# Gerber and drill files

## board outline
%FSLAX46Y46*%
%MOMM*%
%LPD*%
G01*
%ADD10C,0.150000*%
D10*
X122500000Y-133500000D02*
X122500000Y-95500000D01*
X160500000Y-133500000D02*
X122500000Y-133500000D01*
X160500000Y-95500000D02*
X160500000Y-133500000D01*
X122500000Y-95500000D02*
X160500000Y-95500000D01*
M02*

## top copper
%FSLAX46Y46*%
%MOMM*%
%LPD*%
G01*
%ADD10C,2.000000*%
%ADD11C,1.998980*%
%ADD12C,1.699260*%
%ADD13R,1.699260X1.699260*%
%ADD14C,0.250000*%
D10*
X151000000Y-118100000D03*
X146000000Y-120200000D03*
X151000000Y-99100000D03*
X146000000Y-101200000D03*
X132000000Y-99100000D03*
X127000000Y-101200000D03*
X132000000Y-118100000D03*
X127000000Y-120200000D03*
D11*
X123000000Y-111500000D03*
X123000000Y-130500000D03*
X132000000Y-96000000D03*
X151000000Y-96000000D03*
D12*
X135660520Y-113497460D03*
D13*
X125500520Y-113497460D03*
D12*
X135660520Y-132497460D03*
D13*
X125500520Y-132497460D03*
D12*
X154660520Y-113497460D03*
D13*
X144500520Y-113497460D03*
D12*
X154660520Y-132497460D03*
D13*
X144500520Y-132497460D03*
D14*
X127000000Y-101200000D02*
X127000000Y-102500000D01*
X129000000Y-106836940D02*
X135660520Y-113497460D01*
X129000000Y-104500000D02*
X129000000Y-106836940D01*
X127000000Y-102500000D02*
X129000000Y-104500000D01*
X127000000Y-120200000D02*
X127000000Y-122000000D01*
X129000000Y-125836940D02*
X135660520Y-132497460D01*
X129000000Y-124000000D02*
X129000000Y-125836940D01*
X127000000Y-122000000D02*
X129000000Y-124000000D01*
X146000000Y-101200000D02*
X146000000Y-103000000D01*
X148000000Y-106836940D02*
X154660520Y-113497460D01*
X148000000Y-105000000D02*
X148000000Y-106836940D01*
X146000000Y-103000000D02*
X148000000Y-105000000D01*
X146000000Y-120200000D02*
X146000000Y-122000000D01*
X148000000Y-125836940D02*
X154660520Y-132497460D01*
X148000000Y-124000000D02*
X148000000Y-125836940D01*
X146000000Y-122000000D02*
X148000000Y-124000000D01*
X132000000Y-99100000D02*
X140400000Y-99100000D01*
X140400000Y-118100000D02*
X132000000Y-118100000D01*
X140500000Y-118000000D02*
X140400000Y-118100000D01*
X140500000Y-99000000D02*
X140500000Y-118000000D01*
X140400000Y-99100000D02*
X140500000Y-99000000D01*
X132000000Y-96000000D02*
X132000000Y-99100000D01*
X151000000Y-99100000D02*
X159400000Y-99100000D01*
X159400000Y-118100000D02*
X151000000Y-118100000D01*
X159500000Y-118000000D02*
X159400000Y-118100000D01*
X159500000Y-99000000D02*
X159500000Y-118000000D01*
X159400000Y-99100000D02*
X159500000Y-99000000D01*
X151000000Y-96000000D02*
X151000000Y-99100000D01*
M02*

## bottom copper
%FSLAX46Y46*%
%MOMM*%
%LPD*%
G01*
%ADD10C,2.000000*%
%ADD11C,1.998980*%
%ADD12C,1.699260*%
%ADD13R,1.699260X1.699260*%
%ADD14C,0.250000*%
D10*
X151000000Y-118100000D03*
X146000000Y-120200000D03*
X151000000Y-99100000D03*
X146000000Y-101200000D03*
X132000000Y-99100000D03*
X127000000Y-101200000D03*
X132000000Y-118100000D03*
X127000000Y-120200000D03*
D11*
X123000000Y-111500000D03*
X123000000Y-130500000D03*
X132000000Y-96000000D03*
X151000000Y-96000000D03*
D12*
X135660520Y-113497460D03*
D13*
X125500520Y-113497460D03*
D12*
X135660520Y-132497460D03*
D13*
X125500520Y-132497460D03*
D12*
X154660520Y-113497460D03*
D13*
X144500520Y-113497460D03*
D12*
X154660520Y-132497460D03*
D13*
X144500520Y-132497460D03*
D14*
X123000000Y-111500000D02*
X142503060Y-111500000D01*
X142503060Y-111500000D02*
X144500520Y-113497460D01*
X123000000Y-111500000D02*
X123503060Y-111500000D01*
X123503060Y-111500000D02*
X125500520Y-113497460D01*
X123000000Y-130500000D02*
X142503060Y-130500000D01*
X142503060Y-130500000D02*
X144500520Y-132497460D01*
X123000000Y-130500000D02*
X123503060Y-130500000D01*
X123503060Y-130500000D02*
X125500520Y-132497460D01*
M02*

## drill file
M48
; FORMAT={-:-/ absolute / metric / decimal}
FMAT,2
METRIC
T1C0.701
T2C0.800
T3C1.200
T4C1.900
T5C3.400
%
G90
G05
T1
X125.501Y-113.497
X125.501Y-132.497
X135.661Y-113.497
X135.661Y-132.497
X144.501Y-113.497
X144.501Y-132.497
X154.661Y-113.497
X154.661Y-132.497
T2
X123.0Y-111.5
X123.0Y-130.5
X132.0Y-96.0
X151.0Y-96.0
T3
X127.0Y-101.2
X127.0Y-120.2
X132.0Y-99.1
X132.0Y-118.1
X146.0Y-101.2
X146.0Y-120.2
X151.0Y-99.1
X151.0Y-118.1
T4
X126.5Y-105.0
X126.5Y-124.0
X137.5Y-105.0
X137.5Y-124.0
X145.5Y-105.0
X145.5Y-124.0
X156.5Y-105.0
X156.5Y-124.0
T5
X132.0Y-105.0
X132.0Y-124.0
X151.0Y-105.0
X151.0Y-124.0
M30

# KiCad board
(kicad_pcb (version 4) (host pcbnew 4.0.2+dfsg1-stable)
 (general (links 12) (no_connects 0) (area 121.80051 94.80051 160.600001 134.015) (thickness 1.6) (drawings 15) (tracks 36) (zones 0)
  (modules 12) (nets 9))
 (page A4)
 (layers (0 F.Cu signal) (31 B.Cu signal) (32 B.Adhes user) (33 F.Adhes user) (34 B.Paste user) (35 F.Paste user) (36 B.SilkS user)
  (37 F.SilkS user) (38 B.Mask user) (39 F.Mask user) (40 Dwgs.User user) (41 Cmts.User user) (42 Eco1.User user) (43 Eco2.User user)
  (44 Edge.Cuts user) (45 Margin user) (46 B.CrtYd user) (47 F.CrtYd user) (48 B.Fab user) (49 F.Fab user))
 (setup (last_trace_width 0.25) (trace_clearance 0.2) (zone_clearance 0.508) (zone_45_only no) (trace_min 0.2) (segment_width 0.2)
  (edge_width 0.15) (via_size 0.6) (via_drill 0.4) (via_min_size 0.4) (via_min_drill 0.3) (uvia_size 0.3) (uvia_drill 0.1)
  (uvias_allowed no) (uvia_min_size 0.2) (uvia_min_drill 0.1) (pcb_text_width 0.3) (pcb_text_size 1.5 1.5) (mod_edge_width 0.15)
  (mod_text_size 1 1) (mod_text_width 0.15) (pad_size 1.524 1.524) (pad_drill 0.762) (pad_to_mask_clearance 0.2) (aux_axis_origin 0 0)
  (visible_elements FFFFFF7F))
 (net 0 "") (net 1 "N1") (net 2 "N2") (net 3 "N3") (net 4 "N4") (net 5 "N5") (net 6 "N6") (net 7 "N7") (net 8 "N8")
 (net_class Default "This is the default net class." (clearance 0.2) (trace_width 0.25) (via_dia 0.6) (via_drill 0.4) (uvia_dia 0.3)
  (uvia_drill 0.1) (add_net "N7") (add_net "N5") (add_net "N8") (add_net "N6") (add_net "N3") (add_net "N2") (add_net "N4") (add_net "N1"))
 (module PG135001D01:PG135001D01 (layer F.Cu) (at 151 124)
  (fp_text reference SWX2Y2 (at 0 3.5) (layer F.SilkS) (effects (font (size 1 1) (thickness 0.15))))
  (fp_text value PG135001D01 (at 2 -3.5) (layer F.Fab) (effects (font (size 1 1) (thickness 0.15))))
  (pad "" np_thru_hole circle (at 0 0) (size 3.4 3.4) (drill 3.4) (layers *.Cu *.Mask F.SilkS))
  (pad "" np_thru_hole circle (at 5.5 0) (size 1.9 1.9) (drill 1.9) (layers *.Cu *.Mask F.SilkS))
  (pad "" np_thru_hole circle (at -5.5 0) (size 1.9 1.9) (drill 1.9) (layers *.Cu *.Mask F.SilkS))
  (pad 1 thru_hole circle (at 0 -5.9) (size 2 2) (drill 1.2) (layers *.Cu *.Mask F.SilkS) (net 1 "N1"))
  (pad 2 thru_hole circle (at -5 -3.8) (size 2 2) (drill 1.2) (layers *.Cu *.Mask F.SilkS) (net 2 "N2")))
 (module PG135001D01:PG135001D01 (layer F.Cu) (at 151 105)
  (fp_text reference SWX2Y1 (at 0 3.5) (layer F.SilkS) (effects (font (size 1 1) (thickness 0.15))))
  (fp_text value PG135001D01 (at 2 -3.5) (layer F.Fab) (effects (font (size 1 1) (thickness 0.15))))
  (pad "" np_thru_hole circle (at 0 0) (size 3.4 3.4) (drill 3.4) (layers *.Cu *.Mask F.SilkS))
  (pad "" np_thru_hole circle (at 5.5 0) (size 1.9 1.9) (drill 1.9) (layers *.Cu *.Mask F.SilkS))
  (pad "" np_thru_hole circle (at -5.5 0) (size 1.9 1.9) (drill 1.9) (layers *.Cu *.Mask F.SilkS))
  (pad 1 thru_hole circle (at 0 -5.9) (size 2 2) (drill 1.2) (layers *.Cu *.Mask F.SilkS) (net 1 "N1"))
  (pad 2 thru_hole circle (at -5 -3.8) (size 2 2) (drill 1.2) (layers *.Cu *.Mask F.SilkS) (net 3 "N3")))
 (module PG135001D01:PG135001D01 (layer F.Cu) (at 132 105)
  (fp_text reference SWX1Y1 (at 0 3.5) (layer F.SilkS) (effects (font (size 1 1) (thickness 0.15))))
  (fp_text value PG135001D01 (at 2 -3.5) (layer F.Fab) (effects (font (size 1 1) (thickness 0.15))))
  (pad "" np_thru_hole circle (at 0 0) (size 3.4 3.4) (drill 3.4) (layers *.Cu *.Mask F.SilkS))
  (pad "" np_thru_hole circle (at 5.5 0) (size 1.9 1.9) (drill 1.9) (layers *.Cu *.Mask F.SilkS))
  (pad "" np_thru_hole circle (at -5.5 0) (size 1.9 1.9) (drill 1.9) (layers *.Cu *.Mask F.SilkS))
  (pad 1 thru_hole circle (at 0 -5.9) (size 2 2) (drill 1.2) (layers *.Cu *.Mask F.SilkS) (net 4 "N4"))
  (pad 2 thru_hole circle (at -5 -3.8) (size 2 2) (drill 1.2) (layers *.Cu *.Mask F.SilkS) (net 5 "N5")))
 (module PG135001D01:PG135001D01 (layer F.Cu) (at 132 124)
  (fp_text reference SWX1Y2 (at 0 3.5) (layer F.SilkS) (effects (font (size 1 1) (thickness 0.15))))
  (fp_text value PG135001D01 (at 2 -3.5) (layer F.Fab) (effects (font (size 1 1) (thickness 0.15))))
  (pad "" np_thru_hole circle (at 0 0) (size 3.4 3.4) (drill 3.4) (layers *.Cu *.Mask F.SilkS))
  (pad "" np_thru_hole circle (at 5.5 0) (size 1.9 1.9) (drill 1.9) (layers *.Cu *.Mask F.SilkS))
  (pad "" np_thru_hole circle (at -5.5 0) (size 1.9 1.9) (drill 1.9) (layers *.Cu *.Mask F.SilkS))
  (pad 1 thru_hole circle (at 0 -5.9) (size 2 2) (drill 1.2) (layers *.Cu *.Mask F.SilkS) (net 4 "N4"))
  (pad 2 thru_hole circle (at -5 -3.8) (size 2 2) (drill 1.2) (layers *.Cu *.Mask F.SilkS) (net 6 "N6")))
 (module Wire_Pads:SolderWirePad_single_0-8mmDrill (layer F.Cu) (at 123 111.5)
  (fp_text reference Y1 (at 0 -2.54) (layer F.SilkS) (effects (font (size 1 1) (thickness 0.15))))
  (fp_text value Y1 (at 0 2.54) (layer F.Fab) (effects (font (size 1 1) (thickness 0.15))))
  (pad 1 thru_hole circle (at 0 0) (size 1.99898 1.99898) (drill 0.8001) (layers *.Cu *.Mask F.SilkS) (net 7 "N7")))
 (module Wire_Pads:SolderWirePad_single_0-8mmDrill (layer F.Cu) (at 123 130.5)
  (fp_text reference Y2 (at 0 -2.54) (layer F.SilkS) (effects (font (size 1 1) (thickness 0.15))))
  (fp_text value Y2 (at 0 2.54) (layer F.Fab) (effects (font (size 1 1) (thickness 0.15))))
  (pad 1 thru_hole circle (at 0 0) (size 1.99898 1.99898) (drill 0.8001) (layers *.Cu *.Mask F.SilkS) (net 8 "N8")))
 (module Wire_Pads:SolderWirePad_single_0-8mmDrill (layer F.Cu) (at 132 96)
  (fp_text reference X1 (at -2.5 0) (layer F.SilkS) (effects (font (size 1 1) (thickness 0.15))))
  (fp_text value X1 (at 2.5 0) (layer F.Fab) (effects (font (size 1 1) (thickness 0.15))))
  (pad 1 thru_hole circle (at 0 0) (size 1.99898 1.99898) (drill 0.8001) (layers *.Cu *.Mask F.SilkS) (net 4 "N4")))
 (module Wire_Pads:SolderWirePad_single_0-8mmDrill (layer F.Cu) (at 151 96)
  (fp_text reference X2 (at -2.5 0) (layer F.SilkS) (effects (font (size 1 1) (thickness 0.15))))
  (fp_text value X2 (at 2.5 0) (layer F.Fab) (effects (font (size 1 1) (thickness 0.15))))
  (pad 1 thru_hole circle (at 0 0) (size 1.99898 1.99898) (drill 0.8001) (layers *.Cu *.Mask F.SilkS) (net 1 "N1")))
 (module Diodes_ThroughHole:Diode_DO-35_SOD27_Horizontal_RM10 (layer F.Cu) (at 125.5 113.5)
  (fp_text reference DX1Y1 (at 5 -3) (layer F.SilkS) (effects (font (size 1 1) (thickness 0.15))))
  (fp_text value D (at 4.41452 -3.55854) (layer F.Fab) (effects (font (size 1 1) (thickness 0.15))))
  (pad 2 thru_hole circle (at 10.16052 -0.00254 180) (size 1.69926 1.69926) (drill 0.70104) (layers *.Cu *.Mask F.SilkS) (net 5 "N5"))
  (pad 1 thru_hole rect (at 0.00052 -0.00254 180) (size 1.69926 1.69926) (drill 0.70104) (layers *.Cu *.Mask F.SilkS) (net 7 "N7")))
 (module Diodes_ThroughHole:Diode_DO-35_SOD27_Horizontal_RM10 (layer F.Cu) (at 125.5 132.5)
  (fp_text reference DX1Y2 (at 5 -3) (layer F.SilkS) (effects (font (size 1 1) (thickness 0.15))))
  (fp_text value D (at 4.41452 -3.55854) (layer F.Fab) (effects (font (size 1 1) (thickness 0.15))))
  (pad 2 thru_hole circle (at 10.16052 -0.00254 180) (size 1.69926 1.69926) (drill 0.70104) (layers *.Cu *.Mask F.SilkS) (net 6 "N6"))
  (pad 1 thru_hole rect (at 0.00052 -0.00254 180) (size 1.69926 1.69926) (drill 0.70104) (layers *.Cu *.Mask F.SilkS) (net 8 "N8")))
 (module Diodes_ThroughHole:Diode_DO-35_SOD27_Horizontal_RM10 (layer F.Cu) (at 144.5 113.5)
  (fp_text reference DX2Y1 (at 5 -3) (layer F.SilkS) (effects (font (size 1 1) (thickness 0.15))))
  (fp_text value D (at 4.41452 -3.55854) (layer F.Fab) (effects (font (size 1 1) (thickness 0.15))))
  (pad 2 thru_hole circle (at 10.16052 -0.00254 180) (size 1.69926 1.69926) (drill 0.70104) (layers *.Cu *.Mask F.SilkS) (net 3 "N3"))
  (pad 1 thru_hole rect (at 0.00052 -0.00254 180) (size 1.69926 1.69926) (drill 0.70104) (layers *.Cu *.Mask F.SilkS) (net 7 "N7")))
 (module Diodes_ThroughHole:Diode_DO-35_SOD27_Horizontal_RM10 (layer F.Cu) (at 144.5 132.5)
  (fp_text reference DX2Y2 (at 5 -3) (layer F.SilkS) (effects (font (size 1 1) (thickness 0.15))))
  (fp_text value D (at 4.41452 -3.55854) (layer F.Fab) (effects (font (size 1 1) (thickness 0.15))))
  (pad 2 thru_hole circle (at 10.16052 -0.00254 180) (size 1.69926 1.69926) (drill 0.70104) (layers *.Cu *.Mask F.SilkS) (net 2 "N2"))
  (pad 1 thru_hole rect (at 0.00052 -0.00254 180) (size 1.69926 1.69926) (drill 0.70104) (layers *.Cu *.Mask F.SilkS) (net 8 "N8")))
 (gr_line (start 122.5 133.5) (end 122.5 95.5) (angle 90) (layer Edge.Cuts) (width 0.15))
 (gr_line (start 160.5 133.5) (end 122.5 133.5) (angle 90) (layer Edge.Cuts) (width 0.15))
 (gr_line (start 160.5 95.5) (end 160.5 133.5) (angle 90) (layer Edge.Cuts) (width 0.15))
 (gr_line (start 122.5 95.5) (end 160.5 95.5) (angle 90) (layer Edge.Cuts) (width 0.15))
 (segment (start 127 101.2) (end 127 102.5) (width 0.25) (layer F.Cu) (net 5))
 (segment (start 129 106.83694) (end 135.66052 113.49746) (width 0.25) (layer F.Cu) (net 5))
 (segment (start 129 104.5) (end 129 106.83694) (width 0.25) (layer F.Cu) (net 5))
 (segment (start 127 102.5) (end 129 104.5) (width 0.25) (layer F.Cu) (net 5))
 (segment (start 123 111.5) (end 142.50306 111.5) (width 0.25) (layer B.Cu) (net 7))
 (segment (start 142.50306 111.5) (end 144.50052 113.49746) (width 0.25) (layer B.Cu) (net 7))
 (segment (start 123 111.5) (end 123.50306 111.5) (width 0.25) (layer B.Cu) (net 7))
 (segment (start 123.50306 111.5) (end 125.50052 113.49746) (width 0.25) (layer B.Cu) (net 7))
 (segment (start 127 120.2) (end 127 122) (width 0.25) (layer F.Cu) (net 6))
 (segment (start 129 125.83694) (end 135.66052 132.49746) (width 0.25) (layer F.Cu) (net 6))
 (segment (start 129 124) (end 129 125.83694) (width 0.25) (layer F.Cu) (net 6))
 (segment (start 127 122) (end 129 124) (width 0.25) (layer F.Cu) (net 6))
 (segment (start 123 130.5) (end 142.50306 130.5) (width 0.25) (layer B.Cu) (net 8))
 (segment (start 142.50306 130.5) (end 144.50052 132.49746) (width 0.25) (layer B.Cu) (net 8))
 (segment (start 123 130.5) (end 123.50306 130.5) (width 0.25) (layer B.Cu) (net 8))
 (segment (start 123.50306 130.5) (end 125.50052 132.49746) (width 0.25) (layer B.Cu) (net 8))
 (segment (start 146 101.2) (end 146 103) (width 0.25) (layer F.Cu) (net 3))
 (segment (start 148 106.83694) (end 154.66052 113.49746) (width 0.25) (layer F.Cu) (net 3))
 (segment (start 148 105) (end 148 106.83694) (width 0.25) (layer F.Cu) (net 3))
 (segment (start 146 103) (end 148 105) (width 0.25) (layer F.Cu) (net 3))
 (segment (start 146 120.2) (end 146 122) (width 0.25) (layer F.Cu) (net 2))
 (segment (start 148 125.83694) (end 154.66052 132.49746) (width 0.25) (layer F.Cu) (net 2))
 (segment (start 148 124) (end 148 125.83694) (width 0.25) (layer F.Cu) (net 2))
 (segment (start 146 122) (end 148 124) (width 0.25) (layer F.Cu) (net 2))
 (segment (start 132 99.1) (end 140.4 99.1) (width 0.25) (layer F.Cu) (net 4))
 (segment (start 140.4 118.1) (end 132 118.1) (width 0.25) (layer F.Cu) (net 4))
 (segment (start 140.5 118) (end 140.4 118.1) (width 0.25) (layer F.Cu) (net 4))
 (segment (start 140.5 99) (end 140.5 118) (width 0.25) (layer F.Cu) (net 4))
 (segment (start 140.4 99.1) (end 140.5 99) (width 0.25) (layer F.Cu) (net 4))
 (segment (start 132 96) (end 132 99.1) (width 0.25) (layer F.Cu) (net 4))
 (segment (start 151 99.1) (end 159.4 99.1) (width 0.25) (layer F.Cu) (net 1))
 (segment (start 159.4 118.1) (end 151 118.1) (width 0.25) (layer F.Cu) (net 1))
 (segment (start 159.5 118) (end 159.4 118.1) (width 0.25) (layer F.Cu) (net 1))
 (segment (start 159.5 99) (end 159.5 118) (width 0.25) (layer F.Cu) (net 1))
 (segment (start 159.4 99.1) (end 159.5 99) (width 0.25) (layer F.Cu) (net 1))
 (segment (start 151 96) (end 151 99.1) (width 0.25) (layer F.Cu) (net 1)))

